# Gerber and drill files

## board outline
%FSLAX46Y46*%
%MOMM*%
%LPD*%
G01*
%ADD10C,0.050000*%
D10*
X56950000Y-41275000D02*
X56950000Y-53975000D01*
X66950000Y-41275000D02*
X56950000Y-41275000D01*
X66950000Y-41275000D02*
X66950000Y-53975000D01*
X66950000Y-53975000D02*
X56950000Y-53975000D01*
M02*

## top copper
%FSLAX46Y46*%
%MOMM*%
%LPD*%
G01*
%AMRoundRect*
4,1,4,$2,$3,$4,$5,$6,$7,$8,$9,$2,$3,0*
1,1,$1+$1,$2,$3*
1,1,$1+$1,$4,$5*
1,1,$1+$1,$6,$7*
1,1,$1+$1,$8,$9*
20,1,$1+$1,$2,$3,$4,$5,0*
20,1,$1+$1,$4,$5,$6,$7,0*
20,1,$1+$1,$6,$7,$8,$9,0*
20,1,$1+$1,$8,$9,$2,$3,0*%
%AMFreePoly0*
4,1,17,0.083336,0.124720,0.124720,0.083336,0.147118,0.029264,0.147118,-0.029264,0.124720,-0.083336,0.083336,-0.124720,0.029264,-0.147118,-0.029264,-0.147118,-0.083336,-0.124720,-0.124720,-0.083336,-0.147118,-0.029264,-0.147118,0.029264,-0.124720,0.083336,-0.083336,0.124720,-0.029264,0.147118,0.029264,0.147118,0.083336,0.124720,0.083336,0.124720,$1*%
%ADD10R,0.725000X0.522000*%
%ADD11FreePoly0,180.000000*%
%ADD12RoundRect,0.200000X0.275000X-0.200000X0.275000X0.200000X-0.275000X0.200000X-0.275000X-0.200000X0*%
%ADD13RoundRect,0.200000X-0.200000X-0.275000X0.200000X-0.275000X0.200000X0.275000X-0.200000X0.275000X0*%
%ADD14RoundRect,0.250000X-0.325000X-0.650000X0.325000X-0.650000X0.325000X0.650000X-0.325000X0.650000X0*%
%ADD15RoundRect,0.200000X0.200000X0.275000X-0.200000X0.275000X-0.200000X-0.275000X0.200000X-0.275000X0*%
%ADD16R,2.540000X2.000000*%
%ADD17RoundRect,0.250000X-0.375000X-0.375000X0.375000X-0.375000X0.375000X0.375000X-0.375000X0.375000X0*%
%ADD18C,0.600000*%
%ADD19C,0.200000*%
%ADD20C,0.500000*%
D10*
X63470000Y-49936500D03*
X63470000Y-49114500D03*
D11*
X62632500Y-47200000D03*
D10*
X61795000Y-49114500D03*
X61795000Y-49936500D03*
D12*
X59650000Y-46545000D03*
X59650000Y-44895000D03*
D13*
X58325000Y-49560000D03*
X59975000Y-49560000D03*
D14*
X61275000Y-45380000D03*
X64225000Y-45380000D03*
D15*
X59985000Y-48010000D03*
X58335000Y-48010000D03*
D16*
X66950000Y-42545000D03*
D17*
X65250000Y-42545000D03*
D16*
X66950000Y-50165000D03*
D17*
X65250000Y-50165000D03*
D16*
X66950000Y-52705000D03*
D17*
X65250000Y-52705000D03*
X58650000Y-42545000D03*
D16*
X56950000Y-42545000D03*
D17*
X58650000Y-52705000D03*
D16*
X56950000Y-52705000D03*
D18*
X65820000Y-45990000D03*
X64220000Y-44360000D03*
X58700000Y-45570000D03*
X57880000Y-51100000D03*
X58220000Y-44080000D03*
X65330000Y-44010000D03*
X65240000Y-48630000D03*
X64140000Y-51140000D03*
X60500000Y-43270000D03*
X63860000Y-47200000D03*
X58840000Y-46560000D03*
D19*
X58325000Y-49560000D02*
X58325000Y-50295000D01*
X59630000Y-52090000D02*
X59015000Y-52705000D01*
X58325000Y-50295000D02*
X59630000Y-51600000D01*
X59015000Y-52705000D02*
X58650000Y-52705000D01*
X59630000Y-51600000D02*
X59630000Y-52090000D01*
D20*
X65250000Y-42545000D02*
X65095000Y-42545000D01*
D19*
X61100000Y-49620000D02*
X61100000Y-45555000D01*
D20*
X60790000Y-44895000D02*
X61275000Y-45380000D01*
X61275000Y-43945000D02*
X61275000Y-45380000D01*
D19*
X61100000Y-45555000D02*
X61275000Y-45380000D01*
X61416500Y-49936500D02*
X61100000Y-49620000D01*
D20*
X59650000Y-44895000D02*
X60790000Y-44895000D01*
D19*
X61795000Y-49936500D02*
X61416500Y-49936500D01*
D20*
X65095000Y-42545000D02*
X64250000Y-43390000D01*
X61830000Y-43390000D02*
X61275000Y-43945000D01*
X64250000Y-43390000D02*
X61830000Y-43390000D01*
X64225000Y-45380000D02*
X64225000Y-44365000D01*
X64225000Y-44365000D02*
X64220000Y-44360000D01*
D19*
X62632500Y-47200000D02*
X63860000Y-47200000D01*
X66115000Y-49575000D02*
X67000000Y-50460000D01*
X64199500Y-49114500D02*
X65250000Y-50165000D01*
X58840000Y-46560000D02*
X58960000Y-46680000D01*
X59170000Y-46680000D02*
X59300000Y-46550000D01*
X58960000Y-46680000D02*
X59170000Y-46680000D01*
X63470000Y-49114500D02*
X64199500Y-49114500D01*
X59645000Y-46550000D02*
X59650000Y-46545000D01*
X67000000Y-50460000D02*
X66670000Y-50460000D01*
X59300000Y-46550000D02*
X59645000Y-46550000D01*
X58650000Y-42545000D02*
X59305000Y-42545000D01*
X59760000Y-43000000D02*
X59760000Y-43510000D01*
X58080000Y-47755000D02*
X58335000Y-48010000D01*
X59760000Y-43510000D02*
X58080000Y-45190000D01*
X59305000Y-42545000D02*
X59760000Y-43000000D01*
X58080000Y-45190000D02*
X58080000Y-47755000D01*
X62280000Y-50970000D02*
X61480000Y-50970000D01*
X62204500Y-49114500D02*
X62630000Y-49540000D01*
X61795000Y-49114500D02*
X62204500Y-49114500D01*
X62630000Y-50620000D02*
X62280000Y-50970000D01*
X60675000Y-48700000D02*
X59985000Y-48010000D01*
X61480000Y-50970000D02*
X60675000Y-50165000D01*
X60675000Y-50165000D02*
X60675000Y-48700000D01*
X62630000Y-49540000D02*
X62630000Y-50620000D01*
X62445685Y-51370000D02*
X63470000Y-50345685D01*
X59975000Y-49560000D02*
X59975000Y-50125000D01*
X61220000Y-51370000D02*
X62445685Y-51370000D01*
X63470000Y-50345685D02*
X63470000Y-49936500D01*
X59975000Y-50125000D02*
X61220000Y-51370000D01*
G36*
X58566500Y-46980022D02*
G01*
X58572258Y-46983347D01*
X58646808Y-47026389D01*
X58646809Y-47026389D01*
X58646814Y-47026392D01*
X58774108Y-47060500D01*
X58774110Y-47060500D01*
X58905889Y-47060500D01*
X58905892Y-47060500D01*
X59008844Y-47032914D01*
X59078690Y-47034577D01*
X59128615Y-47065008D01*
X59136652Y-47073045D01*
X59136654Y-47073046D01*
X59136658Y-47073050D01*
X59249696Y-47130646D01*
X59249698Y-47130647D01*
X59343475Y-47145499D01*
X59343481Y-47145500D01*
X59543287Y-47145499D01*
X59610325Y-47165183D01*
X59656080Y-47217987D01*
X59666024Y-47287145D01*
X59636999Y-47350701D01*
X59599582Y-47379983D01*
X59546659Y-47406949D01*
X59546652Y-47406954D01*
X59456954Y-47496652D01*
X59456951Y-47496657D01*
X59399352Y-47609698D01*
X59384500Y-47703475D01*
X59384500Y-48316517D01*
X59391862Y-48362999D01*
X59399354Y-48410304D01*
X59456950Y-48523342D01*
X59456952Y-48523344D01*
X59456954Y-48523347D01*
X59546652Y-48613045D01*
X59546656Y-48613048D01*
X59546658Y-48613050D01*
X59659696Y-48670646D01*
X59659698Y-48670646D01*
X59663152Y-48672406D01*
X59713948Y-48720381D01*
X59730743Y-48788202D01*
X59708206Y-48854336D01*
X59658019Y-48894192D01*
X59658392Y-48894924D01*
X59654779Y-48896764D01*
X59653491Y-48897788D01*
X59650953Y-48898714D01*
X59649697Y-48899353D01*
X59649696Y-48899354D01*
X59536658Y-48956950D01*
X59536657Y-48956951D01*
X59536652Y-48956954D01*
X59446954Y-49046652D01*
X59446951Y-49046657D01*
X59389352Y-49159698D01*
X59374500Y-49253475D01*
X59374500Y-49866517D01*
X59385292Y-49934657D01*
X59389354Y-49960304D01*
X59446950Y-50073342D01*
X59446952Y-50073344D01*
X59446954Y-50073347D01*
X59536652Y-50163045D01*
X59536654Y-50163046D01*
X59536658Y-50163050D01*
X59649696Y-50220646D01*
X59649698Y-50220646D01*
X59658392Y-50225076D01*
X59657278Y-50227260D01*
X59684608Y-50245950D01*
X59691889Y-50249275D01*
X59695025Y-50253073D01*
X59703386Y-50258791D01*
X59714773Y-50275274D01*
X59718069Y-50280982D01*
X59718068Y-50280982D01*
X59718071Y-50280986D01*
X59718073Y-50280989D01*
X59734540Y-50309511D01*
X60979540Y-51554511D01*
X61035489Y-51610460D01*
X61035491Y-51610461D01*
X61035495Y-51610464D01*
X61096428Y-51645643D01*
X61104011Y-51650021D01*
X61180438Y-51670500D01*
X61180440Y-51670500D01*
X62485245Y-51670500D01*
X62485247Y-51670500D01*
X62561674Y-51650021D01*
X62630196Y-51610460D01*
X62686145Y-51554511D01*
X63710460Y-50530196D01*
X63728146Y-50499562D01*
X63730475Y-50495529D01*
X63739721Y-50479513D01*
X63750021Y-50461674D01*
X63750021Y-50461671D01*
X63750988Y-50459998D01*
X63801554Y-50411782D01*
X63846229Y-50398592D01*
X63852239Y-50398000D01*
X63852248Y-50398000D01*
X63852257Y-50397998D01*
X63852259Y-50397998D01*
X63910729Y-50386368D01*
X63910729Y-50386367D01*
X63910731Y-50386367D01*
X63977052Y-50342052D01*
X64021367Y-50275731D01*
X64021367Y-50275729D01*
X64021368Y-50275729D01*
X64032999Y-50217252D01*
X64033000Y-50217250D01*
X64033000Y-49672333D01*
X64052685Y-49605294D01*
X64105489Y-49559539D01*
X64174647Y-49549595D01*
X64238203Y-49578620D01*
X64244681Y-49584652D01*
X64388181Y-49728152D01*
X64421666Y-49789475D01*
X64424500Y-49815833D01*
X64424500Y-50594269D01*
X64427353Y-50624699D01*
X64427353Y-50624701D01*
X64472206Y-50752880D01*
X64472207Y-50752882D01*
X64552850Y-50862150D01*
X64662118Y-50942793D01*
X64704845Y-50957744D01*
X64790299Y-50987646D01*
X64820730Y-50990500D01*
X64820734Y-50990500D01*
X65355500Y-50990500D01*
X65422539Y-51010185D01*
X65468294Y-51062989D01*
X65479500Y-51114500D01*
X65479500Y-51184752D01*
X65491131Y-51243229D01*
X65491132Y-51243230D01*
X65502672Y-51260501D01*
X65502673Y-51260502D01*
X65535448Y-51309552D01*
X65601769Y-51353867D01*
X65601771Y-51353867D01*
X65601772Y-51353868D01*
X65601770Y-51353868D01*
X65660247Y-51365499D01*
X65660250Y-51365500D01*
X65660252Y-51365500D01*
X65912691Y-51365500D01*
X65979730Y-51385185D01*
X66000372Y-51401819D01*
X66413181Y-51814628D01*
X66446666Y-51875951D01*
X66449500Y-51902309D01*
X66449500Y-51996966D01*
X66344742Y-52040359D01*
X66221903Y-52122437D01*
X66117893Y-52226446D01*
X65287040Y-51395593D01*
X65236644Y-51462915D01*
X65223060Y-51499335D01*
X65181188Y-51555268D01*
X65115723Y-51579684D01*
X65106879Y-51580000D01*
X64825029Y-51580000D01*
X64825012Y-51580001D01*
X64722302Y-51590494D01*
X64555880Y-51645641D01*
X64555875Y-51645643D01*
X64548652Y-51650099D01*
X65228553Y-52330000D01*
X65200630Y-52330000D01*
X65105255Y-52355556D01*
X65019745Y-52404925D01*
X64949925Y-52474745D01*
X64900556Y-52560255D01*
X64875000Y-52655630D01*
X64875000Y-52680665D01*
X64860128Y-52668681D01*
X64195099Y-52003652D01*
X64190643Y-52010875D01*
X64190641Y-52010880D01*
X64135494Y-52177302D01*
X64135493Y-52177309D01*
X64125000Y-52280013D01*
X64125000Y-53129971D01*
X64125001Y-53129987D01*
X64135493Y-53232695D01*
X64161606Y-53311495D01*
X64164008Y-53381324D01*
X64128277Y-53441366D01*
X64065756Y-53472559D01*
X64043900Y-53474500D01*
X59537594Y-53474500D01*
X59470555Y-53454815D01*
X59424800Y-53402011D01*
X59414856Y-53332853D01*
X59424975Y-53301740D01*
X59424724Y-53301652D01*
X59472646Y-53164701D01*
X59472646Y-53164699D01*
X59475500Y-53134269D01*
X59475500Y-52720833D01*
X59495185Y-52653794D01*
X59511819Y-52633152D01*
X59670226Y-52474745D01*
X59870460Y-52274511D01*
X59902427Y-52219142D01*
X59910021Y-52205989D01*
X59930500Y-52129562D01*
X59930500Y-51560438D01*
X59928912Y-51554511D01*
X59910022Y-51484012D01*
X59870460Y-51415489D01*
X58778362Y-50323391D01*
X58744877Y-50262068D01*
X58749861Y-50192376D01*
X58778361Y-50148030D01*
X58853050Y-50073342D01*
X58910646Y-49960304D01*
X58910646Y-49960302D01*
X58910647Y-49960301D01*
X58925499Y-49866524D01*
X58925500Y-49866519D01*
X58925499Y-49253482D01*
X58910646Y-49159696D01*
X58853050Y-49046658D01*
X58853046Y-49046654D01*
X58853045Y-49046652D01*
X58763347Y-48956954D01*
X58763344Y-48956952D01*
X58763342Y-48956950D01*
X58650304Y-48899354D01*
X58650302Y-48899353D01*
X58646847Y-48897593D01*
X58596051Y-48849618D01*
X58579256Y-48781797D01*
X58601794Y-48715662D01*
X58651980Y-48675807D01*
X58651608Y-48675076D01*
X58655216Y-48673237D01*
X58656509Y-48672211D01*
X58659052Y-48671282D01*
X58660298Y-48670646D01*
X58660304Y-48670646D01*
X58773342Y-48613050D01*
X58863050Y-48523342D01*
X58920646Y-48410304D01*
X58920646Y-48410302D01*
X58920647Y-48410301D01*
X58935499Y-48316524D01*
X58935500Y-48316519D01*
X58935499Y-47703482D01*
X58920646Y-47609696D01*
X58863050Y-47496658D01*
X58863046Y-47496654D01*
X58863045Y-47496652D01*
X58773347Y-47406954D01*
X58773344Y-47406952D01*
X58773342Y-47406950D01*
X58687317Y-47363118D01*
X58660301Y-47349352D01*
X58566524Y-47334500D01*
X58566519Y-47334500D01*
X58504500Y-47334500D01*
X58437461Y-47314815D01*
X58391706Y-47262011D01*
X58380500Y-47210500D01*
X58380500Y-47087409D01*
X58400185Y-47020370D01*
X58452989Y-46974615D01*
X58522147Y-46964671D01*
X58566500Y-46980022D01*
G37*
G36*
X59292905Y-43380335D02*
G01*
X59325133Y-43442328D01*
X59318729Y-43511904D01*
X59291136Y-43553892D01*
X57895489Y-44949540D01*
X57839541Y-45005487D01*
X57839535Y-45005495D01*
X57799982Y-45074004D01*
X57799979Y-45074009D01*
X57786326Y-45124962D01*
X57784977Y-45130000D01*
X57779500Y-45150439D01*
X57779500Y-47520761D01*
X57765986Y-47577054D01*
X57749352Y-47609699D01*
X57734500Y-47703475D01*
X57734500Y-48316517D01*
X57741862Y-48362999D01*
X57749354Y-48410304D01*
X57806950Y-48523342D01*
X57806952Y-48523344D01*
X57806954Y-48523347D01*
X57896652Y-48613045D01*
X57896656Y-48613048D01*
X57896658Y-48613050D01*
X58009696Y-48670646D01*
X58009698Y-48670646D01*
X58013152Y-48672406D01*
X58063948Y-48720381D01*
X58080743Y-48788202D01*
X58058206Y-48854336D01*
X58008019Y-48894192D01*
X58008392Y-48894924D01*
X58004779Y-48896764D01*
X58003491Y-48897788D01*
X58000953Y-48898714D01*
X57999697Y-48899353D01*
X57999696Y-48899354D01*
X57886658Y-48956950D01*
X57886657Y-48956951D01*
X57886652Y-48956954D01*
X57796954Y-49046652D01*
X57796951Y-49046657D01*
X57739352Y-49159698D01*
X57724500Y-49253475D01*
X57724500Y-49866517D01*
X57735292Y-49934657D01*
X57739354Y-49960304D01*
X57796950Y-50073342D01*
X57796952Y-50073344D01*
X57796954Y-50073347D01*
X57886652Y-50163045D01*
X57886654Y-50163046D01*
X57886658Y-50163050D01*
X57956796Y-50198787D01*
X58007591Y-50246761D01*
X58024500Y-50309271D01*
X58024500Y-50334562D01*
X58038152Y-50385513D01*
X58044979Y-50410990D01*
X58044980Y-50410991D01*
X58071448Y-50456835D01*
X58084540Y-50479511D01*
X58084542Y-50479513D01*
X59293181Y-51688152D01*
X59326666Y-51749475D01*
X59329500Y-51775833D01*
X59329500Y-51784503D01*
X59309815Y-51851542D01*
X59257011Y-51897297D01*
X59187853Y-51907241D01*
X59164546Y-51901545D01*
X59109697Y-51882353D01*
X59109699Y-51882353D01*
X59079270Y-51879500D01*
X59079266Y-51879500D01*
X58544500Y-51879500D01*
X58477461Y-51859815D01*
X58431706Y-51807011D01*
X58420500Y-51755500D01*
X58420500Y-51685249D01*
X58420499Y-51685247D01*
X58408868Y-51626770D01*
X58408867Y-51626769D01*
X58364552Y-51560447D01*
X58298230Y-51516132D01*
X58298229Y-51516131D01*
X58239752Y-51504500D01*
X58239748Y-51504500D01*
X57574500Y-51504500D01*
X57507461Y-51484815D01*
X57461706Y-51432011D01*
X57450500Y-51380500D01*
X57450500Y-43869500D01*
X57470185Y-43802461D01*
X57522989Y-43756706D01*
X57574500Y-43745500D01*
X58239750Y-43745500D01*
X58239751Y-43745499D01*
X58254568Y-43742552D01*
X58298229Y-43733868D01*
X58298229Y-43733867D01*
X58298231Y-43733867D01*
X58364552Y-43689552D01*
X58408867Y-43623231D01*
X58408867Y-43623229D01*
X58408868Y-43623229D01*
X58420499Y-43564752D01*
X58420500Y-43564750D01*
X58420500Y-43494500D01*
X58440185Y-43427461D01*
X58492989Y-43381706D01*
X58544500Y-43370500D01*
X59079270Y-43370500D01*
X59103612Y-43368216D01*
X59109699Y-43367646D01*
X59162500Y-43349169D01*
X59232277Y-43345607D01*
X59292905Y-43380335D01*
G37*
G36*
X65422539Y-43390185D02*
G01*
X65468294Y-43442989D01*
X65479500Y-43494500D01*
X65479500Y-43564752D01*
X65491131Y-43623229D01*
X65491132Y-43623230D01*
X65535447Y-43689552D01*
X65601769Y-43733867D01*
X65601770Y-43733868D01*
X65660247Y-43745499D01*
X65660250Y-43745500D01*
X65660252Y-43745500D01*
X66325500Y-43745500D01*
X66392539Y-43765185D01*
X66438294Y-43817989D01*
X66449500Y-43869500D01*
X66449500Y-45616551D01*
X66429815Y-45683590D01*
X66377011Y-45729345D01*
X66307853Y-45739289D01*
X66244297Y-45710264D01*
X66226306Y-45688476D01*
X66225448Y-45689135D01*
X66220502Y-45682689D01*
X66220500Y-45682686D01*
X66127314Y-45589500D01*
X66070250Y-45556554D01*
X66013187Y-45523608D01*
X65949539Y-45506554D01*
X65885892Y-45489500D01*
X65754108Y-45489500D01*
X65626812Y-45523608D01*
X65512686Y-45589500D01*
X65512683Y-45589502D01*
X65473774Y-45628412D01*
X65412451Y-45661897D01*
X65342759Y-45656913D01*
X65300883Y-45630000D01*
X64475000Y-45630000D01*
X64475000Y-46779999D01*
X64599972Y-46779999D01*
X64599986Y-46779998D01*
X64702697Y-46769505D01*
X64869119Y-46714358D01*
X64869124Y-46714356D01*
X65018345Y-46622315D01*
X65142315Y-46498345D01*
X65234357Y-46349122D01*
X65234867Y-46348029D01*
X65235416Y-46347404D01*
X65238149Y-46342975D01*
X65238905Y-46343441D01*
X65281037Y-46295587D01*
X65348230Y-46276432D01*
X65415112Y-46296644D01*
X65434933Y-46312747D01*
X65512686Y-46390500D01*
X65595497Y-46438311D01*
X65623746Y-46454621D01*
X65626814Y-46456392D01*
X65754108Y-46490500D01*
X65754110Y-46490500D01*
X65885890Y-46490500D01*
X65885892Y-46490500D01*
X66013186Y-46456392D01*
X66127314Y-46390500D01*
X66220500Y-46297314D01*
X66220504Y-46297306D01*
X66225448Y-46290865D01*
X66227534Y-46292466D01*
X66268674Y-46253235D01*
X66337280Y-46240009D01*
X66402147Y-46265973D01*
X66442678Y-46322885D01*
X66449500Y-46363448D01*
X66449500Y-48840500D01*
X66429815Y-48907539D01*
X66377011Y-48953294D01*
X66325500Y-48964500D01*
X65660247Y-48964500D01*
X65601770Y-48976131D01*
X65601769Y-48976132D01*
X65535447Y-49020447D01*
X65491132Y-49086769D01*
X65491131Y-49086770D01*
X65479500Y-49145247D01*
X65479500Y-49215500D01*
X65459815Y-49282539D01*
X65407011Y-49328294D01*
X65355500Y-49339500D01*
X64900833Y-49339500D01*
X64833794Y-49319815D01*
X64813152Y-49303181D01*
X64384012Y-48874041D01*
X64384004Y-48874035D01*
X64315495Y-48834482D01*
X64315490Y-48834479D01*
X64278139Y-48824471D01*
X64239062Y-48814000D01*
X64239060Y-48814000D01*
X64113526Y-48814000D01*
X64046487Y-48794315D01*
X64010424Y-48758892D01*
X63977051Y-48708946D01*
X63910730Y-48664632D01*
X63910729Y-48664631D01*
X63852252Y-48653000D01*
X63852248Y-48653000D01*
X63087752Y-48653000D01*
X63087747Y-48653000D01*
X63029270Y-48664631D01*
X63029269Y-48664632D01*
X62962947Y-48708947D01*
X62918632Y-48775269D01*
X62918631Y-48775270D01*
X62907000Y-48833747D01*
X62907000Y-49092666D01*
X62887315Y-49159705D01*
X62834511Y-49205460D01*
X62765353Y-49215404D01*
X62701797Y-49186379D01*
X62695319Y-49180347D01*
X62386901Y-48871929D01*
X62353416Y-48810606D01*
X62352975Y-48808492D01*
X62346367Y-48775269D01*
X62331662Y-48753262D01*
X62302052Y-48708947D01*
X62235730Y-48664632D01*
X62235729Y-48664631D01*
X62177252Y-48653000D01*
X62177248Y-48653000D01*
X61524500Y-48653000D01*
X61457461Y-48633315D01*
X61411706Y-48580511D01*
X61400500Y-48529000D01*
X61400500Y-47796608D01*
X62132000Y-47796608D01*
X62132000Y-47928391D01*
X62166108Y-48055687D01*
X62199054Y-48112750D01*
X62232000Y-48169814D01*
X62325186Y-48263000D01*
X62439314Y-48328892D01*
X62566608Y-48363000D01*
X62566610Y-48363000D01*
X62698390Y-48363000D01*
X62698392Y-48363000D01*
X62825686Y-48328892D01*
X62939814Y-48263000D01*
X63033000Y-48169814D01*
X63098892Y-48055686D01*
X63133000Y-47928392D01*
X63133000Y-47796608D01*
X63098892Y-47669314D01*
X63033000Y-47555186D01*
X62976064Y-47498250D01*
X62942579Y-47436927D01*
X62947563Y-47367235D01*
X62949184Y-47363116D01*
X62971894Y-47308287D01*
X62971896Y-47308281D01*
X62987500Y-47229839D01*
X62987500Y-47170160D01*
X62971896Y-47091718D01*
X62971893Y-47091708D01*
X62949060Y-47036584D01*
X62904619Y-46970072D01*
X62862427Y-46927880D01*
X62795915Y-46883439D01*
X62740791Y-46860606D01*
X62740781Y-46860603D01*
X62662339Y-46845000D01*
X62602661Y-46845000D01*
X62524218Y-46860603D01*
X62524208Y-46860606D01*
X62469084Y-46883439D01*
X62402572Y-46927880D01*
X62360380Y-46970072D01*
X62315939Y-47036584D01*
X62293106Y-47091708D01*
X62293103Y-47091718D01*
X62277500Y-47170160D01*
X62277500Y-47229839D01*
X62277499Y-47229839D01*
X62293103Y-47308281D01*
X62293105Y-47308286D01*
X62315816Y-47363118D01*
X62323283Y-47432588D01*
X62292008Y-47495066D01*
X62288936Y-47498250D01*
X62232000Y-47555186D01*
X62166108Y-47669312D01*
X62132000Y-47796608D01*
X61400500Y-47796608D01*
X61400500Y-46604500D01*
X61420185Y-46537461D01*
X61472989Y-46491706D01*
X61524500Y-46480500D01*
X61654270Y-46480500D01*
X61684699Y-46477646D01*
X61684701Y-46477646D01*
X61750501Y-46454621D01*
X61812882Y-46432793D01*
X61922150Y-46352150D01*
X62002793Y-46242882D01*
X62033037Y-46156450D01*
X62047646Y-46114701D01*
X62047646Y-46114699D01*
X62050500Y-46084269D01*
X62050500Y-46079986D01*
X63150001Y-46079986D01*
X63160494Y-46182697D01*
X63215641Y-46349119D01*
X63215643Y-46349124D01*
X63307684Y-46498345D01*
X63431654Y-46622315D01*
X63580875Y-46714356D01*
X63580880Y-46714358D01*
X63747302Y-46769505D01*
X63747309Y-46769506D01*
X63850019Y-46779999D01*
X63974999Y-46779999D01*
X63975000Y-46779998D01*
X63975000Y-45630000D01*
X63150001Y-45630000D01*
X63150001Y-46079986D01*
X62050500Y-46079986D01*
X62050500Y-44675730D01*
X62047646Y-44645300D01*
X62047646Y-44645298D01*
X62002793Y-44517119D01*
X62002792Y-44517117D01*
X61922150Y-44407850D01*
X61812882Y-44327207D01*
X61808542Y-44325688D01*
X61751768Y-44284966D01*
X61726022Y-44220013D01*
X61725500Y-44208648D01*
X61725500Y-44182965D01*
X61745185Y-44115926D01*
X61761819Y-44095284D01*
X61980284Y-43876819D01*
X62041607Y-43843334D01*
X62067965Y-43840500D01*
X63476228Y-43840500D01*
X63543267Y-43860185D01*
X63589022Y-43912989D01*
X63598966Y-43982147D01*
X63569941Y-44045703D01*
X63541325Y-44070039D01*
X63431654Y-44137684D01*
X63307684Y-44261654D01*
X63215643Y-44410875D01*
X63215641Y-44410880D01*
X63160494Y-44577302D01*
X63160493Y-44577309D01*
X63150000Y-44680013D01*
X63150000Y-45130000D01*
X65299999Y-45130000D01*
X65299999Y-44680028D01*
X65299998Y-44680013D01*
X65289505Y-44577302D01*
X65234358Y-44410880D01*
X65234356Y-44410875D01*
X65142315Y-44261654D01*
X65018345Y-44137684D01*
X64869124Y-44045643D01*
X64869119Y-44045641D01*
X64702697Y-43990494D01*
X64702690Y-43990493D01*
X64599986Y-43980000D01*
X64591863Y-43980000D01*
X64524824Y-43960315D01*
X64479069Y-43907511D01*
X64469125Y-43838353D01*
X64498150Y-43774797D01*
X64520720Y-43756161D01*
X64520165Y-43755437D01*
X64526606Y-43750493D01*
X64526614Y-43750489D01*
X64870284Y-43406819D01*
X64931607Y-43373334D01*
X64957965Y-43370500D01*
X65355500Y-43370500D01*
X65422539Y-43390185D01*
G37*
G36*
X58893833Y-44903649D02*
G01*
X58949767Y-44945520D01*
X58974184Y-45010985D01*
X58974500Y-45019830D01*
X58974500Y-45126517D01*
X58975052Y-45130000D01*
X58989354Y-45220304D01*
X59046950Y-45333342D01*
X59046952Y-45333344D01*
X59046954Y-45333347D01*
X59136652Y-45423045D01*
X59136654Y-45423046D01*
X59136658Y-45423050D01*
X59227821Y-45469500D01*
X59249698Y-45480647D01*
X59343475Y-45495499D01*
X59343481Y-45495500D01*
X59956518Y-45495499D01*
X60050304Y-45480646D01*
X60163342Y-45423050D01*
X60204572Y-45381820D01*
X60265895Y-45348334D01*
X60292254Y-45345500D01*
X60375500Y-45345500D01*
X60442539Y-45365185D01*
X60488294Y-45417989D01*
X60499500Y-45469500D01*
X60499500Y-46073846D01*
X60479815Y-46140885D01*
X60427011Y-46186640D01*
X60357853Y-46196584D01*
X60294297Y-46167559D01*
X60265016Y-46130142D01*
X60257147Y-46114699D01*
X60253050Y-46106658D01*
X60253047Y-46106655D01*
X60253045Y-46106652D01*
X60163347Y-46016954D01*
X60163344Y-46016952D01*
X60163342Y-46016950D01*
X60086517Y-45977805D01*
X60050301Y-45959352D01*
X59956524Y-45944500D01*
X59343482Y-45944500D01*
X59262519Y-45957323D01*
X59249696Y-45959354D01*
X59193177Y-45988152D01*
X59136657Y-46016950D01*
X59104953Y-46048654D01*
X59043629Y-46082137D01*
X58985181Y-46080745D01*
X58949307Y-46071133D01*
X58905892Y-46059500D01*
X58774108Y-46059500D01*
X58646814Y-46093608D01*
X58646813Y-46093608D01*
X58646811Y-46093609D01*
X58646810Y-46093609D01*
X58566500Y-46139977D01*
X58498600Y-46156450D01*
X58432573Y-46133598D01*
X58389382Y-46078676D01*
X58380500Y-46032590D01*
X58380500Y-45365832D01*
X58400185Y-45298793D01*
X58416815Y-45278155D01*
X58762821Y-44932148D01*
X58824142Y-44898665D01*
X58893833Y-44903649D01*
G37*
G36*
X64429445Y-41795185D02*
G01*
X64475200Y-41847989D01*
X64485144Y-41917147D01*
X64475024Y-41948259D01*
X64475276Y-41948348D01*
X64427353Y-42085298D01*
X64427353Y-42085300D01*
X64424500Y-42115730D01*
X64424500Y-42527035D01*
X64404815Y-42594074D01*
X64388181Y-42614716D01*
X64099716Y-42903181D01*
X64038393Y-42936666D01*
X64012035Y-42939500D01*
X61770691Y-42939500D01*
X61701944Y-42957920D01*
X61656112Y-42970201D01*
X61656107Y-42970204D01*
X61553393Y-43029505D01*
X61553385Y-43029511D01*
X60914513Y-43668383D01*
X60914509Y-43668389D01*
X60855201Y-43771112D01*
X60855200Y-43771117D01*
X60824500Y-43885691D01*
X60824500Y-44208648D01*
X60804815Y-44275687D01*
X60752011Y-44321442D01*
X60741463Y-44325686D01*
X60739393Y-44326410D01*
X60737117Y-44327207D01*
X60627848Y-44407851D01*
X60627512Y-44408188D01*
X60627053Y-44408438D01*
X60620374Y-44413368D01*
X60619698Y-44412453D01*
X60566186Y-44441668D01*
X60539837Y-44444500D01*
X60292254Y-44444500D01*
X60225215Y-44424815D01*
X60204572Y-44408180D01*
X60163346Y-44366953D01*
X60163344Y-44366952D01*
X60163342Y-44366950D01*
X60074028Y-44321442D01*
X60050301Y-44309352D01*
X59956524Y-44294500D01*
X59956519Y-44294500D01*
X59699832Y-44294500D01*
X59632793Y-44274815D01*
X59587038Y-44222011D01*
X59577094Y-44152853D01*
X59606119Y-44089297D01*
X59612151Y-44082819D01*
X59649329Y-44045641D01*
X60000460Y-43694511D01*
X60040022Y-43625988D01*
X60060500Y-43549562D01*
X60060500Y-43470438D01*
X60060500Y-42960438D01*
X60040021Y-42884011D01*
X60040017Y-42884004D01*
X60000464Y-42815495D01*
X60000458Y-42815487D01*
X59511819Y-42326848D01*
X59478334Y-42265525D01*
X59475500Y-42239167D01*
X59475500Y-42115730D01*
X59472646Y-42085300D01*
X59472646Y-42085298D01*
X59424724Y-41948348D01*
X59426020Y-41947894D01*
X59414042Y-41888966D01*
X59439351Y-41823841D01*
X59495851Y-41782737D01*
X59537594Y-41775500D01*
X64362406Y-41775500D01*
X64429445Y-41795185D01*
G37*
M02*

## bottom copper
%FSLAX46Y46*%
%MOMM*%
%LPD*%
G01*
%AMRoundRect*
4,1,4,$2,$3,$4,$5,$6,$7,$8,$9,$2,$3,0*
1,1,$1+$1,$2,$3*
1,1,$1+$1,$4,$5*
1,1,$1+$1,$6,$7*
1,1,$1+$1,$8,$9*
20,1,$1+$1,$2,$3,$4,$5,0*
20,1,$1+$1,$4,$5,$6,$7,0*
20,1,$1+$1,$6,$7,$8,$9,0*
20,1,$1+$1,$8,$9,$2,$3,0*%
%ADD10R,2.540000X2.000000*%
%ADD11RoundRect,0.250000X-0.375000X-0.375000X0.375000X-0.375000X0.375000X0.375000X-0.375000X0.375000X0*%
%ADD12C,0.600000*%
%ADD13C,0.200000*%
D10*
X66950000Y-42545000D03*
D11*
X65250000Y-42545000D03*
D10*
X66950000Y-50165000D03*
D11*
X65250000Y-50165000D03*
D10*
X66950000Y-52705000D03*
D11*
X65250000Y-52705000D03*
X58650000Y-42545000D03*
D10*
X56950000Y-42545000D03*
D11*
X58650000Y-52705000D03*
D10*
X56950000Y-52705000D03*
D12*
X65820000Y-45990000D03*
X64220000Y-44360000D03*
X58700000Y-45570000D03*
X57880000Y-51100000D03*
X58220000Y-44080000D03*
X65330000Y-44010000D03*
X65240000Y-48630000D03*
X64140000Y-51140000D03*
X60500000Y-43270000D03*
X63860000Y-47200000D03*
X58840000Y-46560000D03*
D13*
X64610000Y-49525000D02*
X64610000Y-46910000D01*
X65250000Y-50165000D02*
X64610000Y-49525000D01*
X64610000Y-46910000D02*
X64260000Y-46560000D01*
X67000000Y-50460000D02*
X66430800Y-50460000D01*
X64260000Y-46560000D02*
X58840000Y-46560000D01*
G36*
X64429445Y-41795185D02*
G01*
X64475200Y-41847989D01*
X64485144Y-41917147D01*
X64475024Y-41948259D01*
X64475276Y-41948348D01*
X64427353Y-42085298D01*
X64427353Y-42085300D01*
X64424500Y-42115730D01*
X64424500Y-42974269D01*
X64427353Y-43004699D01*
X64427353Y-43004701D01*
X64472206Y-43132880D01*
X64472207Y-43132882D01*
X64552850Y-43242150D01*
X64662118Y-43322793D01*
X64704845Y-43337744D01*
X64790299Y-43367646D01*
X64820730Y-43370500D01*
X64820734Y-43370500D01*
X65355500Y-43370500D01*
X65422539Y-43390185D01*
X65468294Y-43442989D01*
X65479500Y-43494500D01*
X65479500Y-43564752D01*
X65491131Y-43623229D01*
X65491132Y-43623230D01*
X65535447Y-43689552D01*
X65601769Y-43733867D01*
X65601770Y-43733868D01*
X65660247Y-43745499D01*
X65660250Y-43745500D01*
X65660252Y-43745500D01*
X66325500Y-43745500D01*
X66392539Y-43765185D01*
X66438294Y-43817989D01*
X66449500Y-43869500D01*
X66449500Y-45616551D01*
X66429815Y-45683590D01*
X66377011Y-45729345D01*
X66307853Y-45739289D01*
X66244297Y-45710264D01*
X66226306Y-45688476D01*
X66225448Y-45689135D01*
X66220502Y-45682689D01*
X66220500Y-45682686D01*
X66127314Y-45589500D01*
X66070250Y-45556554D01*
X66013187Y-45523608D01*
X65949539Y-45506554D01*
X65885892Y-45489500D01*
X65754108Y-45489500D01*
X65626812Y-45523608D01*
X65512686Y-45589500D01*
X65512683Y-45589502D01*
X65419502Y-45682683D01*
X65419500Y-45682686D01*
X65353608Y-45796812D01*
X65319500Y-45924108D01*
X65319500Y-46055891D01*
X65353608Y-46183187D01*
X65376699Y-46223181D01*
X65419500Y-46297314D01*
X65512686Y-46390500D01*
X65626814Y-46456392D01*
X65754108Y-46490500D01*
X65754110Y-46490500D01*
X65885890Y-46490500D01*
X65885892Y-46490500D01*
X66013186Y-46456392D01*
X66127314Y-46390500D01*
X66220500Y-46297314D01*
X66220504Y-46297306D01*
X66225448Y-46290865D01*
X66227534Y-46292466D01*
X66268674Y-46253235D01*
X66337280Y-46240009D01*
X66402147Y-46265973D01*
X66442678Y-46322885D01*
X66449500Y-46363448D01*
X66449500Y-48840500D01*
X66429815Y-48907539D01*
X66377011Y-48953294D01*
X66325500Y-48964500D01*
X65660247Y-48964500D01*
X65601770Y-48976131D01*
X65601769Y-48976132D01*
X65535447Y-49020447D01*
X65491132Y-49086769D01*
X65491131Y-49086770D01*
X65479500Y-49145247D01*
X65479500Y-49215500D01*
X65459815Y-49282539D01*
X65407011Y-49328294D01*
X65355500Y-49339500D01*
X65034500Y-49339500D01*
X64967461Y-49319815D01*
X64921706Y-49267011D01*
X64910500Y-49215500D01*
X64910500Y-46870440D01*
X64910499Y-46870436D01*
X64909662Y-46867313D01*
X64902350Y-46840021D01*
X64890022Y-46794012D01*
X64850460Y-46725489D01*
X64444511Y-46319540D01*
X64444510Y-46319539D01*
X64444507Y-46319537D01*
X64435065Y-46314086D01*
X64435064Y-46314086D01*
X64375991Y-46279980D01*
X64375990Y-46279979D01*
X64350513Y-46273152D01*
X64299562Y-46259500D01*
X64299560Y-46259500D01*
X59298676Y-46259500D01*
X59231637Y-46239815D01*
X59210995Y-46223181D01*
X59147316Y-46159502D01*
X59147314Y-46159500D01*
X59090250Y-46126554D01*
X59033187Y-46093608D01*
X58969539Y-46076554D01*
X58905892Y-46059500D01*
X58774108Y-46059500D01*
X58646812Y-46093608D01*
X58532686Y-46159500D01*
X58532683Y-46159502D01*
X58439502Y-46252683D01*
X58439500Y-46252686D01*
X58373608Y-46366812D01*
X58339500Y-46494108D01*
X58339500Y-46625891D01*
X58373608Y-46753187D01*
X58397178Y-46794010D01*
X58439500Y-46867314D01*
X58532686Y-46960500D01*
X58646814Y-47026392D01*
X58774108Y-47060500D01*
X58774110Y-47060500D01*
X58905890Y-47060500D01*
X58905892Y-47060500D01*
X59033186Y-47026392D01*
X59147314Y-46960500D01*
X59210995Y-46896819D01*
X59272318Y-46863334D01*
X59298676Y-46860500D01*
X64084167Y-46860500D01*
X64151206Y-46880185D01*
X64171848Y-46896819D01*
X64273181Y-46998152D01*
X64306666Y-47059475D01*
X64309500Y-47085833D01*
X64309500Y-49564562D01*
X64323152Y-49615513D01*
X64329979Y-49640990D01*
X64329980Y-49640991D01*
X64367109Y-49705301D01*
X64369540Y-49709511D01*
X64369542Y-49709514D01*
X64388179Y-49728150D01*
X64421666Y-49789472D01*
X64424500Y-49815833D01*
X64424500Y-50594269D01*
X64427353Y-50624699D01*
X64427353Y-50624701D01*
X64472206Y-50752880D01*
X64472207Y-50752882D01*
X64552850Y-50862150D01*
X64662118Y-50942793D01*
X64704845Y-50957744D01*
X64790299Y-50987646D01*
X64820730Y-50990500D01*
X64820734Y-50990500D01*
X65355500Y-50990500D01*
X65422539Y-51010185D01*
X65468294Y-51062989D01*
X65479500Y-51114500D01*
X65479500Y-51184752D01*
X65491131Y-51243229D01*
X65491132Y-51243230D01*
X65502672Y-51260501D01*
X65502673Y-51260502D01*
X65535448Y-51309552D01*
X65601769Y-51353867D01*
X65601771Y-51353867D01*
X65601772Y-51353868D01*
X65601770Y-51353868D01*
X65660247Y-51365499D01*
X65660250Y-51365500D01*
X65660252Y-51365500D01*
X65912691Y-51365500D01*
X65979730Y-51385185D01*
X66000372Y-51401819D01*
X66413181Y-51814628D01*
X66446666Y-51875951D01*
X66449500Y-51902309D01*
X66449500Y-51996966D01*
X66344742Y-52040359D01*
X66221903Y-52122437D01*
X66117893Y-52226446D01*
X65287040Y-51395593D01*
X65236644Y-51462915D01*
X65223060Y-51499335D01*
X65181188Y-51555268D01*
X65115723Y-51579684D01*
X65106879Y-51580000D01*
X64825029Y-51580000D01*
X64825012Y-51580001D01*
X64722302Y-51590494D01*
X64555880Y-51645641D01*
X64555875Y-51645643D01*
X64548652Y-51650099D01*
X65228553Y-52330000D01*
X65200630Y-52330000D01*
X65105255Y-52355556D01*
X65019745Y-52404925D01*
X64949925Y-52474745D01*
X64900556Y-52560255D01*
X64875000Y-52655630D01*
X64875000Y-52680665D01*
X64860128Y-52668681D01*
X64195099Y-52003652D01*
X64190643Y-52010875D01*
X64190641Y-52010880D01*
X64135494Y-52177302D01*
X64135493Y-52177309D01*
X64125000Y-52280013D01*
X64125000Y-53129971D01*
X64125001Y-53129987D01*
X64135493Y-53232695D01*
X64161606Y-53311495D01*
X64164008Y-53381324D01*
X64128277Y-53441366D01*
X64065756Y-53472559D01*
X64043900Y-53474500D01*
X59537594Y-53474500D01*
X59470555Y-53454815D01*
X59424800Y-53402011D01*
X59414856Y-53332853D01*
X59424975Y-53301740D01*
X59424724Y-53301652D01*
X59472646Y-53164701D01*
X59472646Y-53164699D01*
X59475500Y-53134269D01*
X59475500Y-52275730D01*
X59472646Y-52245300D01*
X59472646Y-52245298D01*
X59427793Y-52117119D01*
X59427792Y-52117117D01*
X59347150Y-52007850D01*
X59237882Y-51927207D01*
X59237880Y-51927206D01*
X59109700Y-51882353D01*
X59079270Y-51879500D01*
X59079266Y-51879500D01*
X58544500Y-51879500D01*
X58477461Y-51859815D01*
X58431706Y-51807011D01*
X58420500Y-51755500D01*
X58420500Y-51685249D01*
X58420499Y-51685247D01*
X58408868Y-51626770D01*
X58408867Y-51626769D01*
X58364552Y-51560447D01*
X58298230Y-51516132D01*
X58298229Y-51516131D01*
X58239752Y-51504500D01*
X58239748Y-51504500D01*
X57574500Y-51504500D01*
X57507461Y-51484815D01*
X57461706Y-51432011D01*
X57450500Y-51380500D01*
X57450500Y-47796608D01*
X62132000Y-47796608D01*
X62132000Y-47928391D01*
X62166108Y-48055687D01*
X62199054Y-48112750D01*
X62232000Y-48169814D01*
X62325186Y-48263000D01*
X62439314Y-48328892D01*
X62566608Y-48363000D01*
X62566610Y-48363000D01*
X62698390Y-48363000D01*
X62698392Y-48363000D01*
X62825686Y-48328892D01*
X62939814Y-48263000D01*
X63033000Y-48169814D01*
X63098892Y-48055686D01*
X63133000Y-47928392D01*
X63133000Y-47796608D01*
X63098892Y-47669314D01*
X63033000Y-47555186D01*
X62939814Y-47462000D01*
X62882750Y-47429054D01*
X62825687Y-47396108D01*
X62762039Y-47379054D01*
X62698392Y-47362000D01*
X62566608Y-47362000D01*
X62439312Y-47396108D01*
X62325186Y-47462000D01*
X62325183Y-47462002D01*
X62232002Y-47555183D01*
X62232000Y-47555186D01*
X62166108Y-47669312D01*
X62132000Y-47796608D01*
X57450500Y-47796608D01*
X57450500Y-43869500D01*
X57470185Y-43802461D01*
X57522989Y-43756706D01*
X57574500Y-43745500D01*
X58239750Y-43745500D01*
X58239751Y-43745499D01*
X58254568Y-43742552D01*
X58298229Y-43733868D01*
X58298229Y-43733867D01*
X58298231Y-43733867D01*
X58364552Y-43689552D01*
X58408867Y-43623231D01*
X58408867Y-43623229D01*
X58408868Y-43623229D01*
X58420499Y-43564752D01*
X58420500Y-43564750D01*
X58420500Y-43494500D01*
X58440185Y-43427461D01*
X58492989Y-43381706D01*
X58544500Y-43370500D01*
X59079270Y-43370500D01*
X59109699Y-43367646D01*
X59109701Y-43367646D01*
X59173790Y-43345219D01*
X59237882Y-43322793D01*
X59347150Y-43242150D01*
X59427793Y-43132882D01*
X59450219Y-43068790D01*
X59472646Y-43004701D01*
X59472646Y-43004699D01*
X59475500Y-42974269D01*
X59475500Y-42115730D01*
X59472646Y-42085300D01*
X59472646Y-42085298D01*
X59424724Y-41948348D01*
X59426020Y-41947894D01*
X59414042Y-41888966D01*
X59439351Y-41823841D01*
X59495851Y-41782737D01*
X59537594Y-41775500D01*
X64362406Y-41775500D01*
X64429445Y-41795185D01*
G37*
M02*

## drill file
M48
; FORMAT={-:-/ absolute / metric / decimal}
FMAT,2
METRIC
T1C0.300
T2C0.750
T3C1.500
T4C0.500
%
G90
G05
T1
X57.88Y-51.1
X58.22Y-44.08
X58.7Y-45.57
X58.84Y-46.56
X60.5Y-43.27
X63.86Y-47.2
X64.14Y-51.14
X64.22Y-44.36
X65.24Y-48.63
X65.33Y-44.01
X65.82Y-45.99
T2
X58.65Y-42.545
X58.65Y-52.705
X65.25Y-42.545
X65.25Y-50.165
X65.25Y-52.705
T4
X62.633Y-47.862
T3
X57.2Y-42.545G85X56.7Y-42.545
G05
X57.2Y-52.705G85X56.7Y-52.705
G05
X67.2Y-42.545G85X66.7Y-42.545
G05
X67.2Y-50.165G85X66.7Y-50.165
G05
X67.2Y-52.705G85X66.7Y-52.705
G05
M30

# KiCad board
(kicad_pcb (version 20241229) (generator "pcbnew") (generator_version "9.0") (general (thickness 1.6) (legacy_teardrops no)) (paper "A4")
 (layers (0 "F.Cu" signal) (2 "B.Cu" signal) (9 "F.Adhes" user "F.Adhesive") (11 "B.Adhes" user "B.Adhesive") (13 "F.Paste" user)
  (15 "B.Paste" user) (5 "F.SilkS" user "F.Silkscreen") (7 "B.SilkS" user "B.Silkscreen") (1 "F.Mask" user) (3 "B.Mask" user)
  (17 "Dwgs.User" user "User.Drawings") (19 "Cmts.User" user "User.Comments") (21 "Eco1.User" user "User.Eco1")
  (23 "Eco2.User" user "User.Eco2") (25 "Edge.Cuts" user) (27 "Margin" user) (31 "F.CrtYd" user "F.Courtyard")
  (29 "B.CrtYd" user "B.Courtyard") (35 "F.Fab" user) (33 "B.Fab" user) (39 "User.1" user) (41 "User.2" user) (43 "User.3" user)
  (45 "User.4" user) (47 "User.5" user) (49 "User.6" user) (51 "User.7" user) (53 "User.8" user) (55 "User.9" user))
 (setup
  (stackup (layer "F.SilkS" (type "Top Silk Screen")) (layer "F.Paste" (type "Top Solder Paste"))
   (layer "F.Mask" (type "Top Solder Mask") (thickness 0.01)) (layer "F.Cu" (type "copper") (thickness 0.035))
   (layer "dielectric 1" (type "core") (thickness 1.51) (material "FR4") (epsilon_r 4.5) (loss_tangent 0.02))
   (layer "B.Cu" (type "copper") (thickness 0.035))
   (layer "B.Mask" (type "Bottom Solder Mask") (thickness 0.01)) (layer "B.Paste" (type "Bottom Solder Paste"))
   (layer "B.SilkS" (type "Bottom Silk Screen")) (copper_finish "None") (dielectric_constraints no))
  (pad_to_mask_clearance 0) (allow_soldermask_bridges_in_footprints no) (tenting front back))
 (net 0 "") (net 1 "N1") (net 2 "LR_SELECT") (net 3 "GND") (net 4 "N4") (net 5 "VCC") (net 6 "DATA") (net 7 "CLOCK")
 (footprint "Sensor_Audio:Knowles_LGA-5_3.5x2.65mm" (layer "F.Cu") (at 62.6325 48.6325 180)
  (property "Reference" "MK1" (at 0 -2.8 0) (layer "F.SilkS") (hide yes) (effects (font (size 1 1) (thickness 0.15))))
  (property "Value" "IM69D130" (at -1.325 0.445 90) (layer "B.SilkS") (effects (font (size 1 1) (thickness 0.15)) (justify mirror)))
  (pad "" np_thru_hole circle (at 0 0.77 180) (size 0.5 0.5) (drill 0.5) (layers "*.Cu" "*.Mask"))
  (pad "1" smd rect (at -0.8375 -1.304 180) (size 0.725 0.522) (layers "F.Cu" "F.Mask" "F.Paste") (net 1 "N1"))
  (pad "2" smd rect (at -0.8375 -0.482 180) (size 0.725 0.522) (layers "F.Cu" "F.Mask" "F.Paste") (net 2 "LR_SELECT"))
  (pad "3" smd custom (at 0 1.4325 180) (size 0.3 0.3) (layers "F.Cu" "F.Mask") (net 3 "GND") (zone_connect 0)
   (options (clearance outline) (anchor circle)) (primitives))
  (pad "4" smd rect (at 0.8375 -0.482 180) (size 0.725 0.522) (layers "F.Cu" "F.Mask" "F.Paste") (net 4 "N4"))
  (pad "5" smd rect (at 0.8375 -1.304 180) (size 0.725 0.522) (layers "F.Cu" "F.Mask" "F.Paste") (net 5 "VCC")))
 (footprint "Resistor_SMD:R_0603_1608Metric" (layer "F.Cu") (at 59.65 45.72 90)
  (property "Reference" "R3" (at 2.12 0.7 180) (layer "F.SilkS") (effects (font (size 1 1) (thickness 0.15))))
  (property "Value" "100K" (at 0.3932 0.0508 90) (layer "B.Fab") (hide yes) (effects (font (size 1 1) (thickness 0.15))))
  (pad "1" smd roundrect (at -0.825 0 90) (size 0.8 0.95) (layers "F.Cu" "F.Mask" "F.Paste") (roundrect_rratio 0.25) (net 2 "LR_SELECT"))
  (pad "2" smd roundrect (at 0.825 0 90) (size 0.8 0.95) (layers "F.Cu" "F.Mask" "F.Paste") (roundrect_rratio 0.25) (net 5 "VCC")))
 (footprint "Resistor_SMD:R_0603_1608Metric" (layer "F.Cu") (at 59.15 49.56)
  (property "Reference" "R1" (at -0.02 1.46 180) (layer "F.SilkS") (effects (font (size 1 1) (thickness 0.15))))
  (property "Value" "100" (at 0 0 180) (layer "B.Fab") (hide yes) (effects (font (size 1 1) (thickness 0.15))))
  (pad "1" smd roundrect (at -0.825 0) (size 0.8 0.95) (layers "F.Cu" "F.Mask" "F.Paste") (roundrect_rratio 0.25) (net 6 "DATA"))
  (pad "2" smd roundrect (at 0.825 0) (size 0.8 0.95) (layers "F.Cu" "F.Mask" "F.Paste") (roundrect_rratio 0.25) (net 1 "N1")))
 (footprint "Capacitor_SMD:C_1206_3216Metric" (layer "F.Cu") (at 62.75 45.38)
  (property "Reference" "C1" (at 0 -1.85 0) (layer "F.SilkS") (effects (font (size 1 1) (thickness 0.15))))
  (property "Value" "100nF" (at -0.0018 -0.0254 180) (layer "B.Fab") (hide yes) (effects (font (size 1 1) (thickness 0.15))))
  (pad "1" smd roundrect (at -1.475 0) (size 1.15 1.8) (layers "F.Cu" "F.Mask" "F.Paste") (roundrect_rratio 0.217391) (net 5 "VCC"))
  (pad "2" smd roundrect (at 1.475 0) (size 1.15 1.8) (layers "F.Cu" "F.Mask" "F.Paste") (roundrect_rratio 0.217391) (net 3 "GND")))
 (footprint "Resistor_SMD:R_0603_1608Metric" (layer "F.Cu") (at 59.16 48.01 180)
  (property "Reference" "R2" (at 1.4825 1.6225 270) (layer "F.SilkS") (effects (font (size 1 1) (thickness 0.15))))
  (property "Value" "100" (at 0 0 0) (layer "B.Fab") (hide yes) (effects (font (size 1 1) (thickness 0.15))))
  (pad "1" smd roundrect (at -0.825 0 180) (size 0.8 0.95) (layers "F.Cu" "F.Mask" "F.Paste") (roundrect_rratio 0.25) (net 4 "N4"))
  (pad "2" smd roundrect (at 0.825 0 180) (size 0.8 0.95) (layers "F.Cu" "F.Mask" "F.Paste") (roundrect_rratio 0.25) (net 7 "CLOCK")))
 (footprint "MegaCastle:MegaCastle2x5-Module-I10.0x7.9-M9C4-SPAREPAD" (layer "B.Cu") (at 61.95 47.625 180)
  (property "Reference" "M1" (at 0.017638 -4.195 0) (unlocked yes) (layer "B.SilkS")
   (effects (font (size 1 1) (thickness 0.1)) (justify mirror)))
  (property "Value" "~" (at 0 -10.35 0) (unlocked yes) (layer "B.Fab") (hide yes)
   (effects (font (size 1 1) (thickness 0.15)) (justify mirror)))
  (fp_line (start 5 6.35) (end 5 -6.35) (stroke (width 0.05) (type default)) (layer "Edge.Cuts"))
  (fp_line (start -5 6.35) (end 5 6.35) (stroke (width 0.05) (type default)) (layer "Edge.Cuts"))
  (fp_line (start -5 6.35) (end -5 -6.35) (stroke (width 0.05) (type default)) (layer "Edge.Cuts"))
  (fp_line (start -5 -6.35) (end 5 -6.35) (stroke (width 0.05) (type default)) (layer "Edge.Cuts"))
  (pad "1" thru_hole rect (at -5 5.08 180) (size 2.54 2) (drill oval 2 1.5) (layers "*.Cu" "*.Mask") (remove_unused_layers no) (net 5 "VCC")
   (thermal_bridge_angle 45))
  (pad "1" thru_hole roundrect (at -3.3 5.08) (size 1.25 1.25) (drill 0.75) (layers "*.Cu" "*.Mask") (remove_unused_layers no)
   (roundrect_rratio 0.2) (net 5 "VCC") (thermal_bridge_angle 45))
  (pad "4" thru_hole rect (at -5 -2.54 180) (size 2.54 2) (drill oval 2 1.5) (layers "*.Cu" "*.Mask") (remove_unused_layers no)
   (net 2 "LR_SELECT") (thermal_bridge_angle 45))
  (pad "4" thru_hole roundrect (at -3.3 -2.54) (size 1.25 1.25) (drill 0.75) (layers "*.Cu" "*.Mask") (remove_unused_layers no)
   (roundrect_rratio 0.2) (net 2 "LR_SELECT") (thermal_bridge_angle 45))
  (pad "5" thru_hole rect (at -5 -5.08 180) (size 2.54 2) (drill oval 2 1.5) (layers "*.Cu" "*.Mask") (remove_unused_layers no)
   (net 3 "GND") (thermal_bridge_angle 45))
  (pad "5" thru_hole roundrect (at -3.3 -5.08) (size 1.25 1.25) (drill 0.75) (layers "*.Cu" "*.Mask") (remove_unused_layers no)
   (roundrect_rratio 0.2) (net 3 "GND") (thermal_bridge_angle 45))
  (pad "6" thru_hole roundrect (at 3.3 5.08) (size 1.25 1.25) (drill 0.75) (layers "*.Cu" "*.Mask") (remove_unused_layers no)
   (roundrect_rratio 0.2) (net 7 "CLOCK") (thermal_bridge_angle 45))
  (pad "6" thru_hole rect (at 5 5.08 180) (size 2.54 2) (drill oval 2 1.5) (layers "*.Cu" "*.Mask") (remove_unused_layers no)
   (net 7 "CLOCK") (thermal_bridge_angle 45))
  (pad "10" thru_hole roundrect (at 3.3 -5.08) (size 1.25 1.25) (drill 0.75) (layers "*.Cu" "*.Mask") (remove_unused_layers no)
   (roundrect_rratio 0.2) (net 6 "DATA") (thermal_bridge_angle 45))
  (pad "10" thru_hole rect (at 5 -5.08 180) (size 2.54 2) (drill oval 2 1.5) (layers "*.Cu" "*.Mask") (remove_unused_layers no)
   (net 6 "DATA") (thermal_bridge_angle 45))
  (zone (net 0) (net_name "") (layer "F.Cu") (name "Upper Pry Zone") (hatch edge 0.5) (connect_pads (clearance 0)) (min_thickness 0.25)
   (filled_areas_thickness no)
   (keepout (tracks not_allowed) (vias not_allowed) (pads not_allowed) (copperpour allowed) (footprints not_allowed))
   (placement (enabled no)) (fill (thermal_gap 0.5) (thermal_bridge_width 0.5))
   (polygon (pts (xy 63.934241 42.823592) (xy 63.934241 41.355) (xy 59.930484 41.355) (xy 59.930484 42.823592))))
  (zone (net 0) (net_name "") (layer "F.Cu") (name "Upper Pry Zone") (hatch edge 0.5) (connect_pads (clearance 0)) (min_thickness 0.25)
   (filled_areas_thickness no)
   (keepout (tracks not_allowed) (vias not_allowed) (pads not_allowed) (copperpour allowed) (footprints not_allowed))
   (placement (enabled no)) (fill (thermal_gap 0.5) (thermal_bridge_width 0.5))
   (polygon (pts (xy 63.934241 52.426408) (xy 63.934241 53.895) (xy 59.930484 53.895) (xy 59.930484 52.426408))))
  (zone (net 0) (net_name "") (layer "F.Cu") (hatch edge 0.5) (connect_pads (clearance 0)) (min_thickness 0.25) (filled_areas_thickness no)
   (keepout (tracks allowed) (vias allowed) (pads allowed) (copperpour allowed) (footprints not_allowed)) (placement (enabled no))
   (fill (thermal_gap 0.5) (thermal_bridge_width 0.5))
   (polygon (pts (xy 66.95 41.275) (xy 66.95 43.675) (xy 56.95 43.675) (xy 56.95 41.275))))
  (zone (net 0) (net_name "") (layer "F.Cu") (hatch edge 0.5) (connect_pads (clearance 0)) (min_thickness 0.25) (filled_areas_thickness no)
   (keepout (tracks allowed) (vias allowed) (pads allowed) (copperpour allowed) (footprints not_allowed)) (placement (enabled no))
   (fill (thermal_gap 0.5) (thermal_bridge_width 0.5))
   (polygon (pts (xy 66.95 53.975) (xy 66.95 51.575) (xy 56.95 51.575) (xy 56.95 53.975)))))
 (via (at 65.82 45.99) (size 0.6) (drill 0.3) (layers "F.Cu" "B.Cu") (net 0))
 (segment (start 58.325 49.56) (end 58.325 50.295) (width 0.2) (layer "F.Cu") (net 6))
 (segment (start 59.63 52.09) (end 59.015 52.705) (width 0.2) (layer "F.Cu") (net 6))
 (segment (start 58.325 50.295) (end 59.63 51.6) (width 0.2) (layer "F.Cu") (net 6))
 (segment (start 59.015 52.705) (end 58.65 52.705) (width 0.2) (layer "F.Cu") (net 6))
 (segment (start 59.63 51.6) (end 59.63 52.09) (width 0.2) (layer "F.Cu") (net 6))
 (segment (start 65.25 42.545) (end 65.095 42.545) (width 0.5) (layer "F.Cu") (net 5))
 (segment (start 61.1 49.62) (end 61.1 45.555) (width 0.2) (layer "F.Cu") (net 5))
 (segment (start 60.79 44.895) (end 61.275 45.38) (width 0.5) (layer "F.Cu") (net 5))
 (segment (start 61.275 43.945) (end 61.275 45.38) (width 0.5) (layer "F.Cu") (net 5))
 (segment (start 61.1 45.555) (end 61.275 45.38) (width 0.2) (layer "F.Cu") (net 5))
 (segment (start 61.4165 49.9365) (end 61.1 49.62) (width 0.2) (layer "F.Cu") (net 5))
 (segment (start 59.65 44.895) (end 60.79 44.895) (width 0.5) (layer "F.Cu") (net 5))
 (segment (start 61.795 49.9365) (end 61.4165 49.9365) (width 0.2) (layer "F.Cu") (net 5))
 (segment (start 65.095 42.545) (end 64.25 43.39) (width 0.5) (layer "F.Cu") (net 5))
 (segment (start 61.83 43.39) (end 61.275 43.945) (width 0.5) (layer "F.Cu") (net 5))
 (segment (start 64.25 43.39) (end 61.83 43.39) (width 0.5) (layer "F.Cu") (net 5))
 (segment (start 64.225 45.38) (end 64.225 44.365) (width 0.5) (layer "F.Cu") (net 3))
 (segment (start 64.225 44.365) (end 64.22 44.36) (width 0.5) (layer "F.Cu") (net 3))
 (segment (start 62.6325 47.2) (end 63.86 47.2) (width 0.2) (layer "F.Cu") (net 3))
 (via (at 64.22 44.36) (size 0.6) (drill 0.3) (layers "F.Cu" "B.Cu") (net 3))
 (via (at 58.7 45.57) (size 0.6) (drill 0.3) (layers "F.Cu" "B.Cu") (free yes) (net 3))
 (via (at 57.88 51.1) (size 0.6) (drill 0.3) (layers "F.Cu" "B.Cu") (free yes) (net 3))
 (via (at 58.22 44.08) (size 0.6) (drill 0.3) (layers "F.Cu" "B.Cu") (free yes) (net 3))
 (via (at 65.33 44.01) (size 0.6) (drill 0.3) (layers "F.Cu" "B.Cu") (free yes) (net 3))
 (via (at 65.24 48.63) (size 0.6) (drill 0.3) (layers "F.Cu" "B.Cu") (free yes) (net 3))
 (via (at 64.14 51.14) (size 0.6) (drill 0.3) (layers "F.Cu" "B.Cu") (free yes) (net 3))
 (via (at 60.5 43.27) (size 0.6) (drill 0.3) (layers "F.Cu" "B.Cu") (free yes) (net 3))
 (via (at 63.86 47.2) (size 0.6) (drill 0.3) (layers "F.Cu" "B.Cu") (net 3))
 (segment (start 66.115 49.575) (end 67 50.46) (width 0.2) (layer "F.Cu") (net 2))
 (segment (start 64.1995 49.1145) (end 65.25 50.165) (width 0.2) (layer "F.Cu") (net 2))
 (segment (start 58.84 46.56) (end 58.96 46.68) (width 0.2) (layer "F.Cu") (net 2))
 (segment (start 59.17 46.68) (end 59.3 46.55) (width 0.2) (layer "F.Cu") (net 2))
 (segment (start 58.96 46.68) (end 59.17 46.68) (width 0.2) (layer "F.Cu") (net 2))
 (segment (start 63.47 49.1145) (end 64.1995 49.1145) (width 0.2) (layer "F.Cu") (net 2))
 (segment (start 59.645 46.55) (end 59.65 46.545) (width 0.2) (layer "F.Cu") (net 2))
 (segment (start 67 50.46) (end 66.67 50.46) (width 0.2) (layer "F.Cu") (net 2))
 (segment (start 59.3 46.55) (end 59.645 46.55) (width 0.2) (layer "F.Cu") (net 2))
 (via (at 58.84 46.56) (size 0.6) (drill 0.3) (layers "F.Cu" "B.Cu") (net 2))
 (segment (start 64.61 49.525) (end 64.61 46.91) (width 0.2) (layer "B.Cu") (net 2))
 (segment (start 65.25 50.165) (end 64.61 49.525) (width 0.2) (layer "B.Cu") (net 2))
 (segment (start 64.61 46.91) (end 64.26 46.56) (width 0.2) (layer "B.Cu") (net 2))
 (segment (start 67 50.46) (end 66.4308 50.46) (width 0.2) (layer "B.Cu") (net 2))
 (segment (start 64.26 46.56) (end 58.84 46.56) (width 0.2) (layer "B.Cu") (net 2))
 (segment (start 58.65 42.545) (end 59.305 42.545) (width 0.2) (layer "F.Cu") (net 7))
 (segment (start 59.76 43) (end 59.76 43.51) (width 0.2) (layer "F.Cu") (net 7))
 (segment (start 58.08 47.755) (end 58.335 48.01) (width 0.2) (layer "F.Cu") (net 7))
 (segment (start 59.76 43.51) (end 58.08 45.19) (width 0.2) (layer "F.Cu") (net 7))
 (segment (start 59.305 42.545) (end 59.76 43) (width 0.2) (layer "F.Cu") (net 7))
 (segment (start 58.08 45.19) (end 58.08 47.755) (width 0.2) (layer "F.Cu") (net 7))
 (segment (start 62.28 50.97) (end 61.48 50.97) (width 0.2) (layer "F.Cu") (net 4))
 (segment (start 62.2045 49.1145) (end 62.63 49.54) (width 0.2) (layer "F.Cu") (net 4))
 (segment (start 61.795 49.1145) (end 62.2045 49.1145) (width 0.2) (layer "F.Cu") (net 4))
 (segment (start 62.63 50.62) (end 62.28 50.97) (width 0.2) (layer "F.Cu") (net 4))
 (segment (start 60.675 48.7) (end 59.985 48.01) (width 0.2) (layer "F.Cu") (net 4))
 (segment (start 61.48 50.97) (end 60.675 50.165) (width 0.2) (layer "F.Cu") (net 4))
 (segment (start 60.675 50.165) (end 60.675 48.7) (width 0.2) (layer "F.Cu") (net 4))
 (segment (start 62.63 49.54) (end 62.63 50.62) (width 0.2) (layer "F.Cu") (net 4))
 (segment (start 62.445685 51.37) (end 63.47 50.345685) (width 0.2) (layer "F.Cu") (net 1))
 (segment (start 59.975 49.56) (end 59.975 50.125) (width 0.2) (layer "F.Cu") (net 1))
 (segment (start 61.22 51.37) (end 62.445685 51.37) (width 0.2) (layer "F.Cu") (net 1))
 (segment (start 63.47 50.345685) (end 63.47 49.9365) (width 0.2) (layer "F.Cu") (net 1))
 (segment (start 59.975 50.125) (end 61.22 51.37) (width 0.2) (layer "F.Cu") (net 1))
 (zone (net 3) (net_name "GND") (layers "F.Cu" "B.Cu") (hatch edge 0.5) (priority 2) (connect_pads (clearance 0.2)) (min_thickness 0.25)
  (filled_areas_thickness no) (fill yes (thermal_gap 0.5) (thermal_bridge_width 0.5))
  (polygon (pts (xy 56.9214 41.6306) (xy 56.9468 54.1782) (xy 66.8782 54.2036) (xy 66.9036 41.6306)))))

